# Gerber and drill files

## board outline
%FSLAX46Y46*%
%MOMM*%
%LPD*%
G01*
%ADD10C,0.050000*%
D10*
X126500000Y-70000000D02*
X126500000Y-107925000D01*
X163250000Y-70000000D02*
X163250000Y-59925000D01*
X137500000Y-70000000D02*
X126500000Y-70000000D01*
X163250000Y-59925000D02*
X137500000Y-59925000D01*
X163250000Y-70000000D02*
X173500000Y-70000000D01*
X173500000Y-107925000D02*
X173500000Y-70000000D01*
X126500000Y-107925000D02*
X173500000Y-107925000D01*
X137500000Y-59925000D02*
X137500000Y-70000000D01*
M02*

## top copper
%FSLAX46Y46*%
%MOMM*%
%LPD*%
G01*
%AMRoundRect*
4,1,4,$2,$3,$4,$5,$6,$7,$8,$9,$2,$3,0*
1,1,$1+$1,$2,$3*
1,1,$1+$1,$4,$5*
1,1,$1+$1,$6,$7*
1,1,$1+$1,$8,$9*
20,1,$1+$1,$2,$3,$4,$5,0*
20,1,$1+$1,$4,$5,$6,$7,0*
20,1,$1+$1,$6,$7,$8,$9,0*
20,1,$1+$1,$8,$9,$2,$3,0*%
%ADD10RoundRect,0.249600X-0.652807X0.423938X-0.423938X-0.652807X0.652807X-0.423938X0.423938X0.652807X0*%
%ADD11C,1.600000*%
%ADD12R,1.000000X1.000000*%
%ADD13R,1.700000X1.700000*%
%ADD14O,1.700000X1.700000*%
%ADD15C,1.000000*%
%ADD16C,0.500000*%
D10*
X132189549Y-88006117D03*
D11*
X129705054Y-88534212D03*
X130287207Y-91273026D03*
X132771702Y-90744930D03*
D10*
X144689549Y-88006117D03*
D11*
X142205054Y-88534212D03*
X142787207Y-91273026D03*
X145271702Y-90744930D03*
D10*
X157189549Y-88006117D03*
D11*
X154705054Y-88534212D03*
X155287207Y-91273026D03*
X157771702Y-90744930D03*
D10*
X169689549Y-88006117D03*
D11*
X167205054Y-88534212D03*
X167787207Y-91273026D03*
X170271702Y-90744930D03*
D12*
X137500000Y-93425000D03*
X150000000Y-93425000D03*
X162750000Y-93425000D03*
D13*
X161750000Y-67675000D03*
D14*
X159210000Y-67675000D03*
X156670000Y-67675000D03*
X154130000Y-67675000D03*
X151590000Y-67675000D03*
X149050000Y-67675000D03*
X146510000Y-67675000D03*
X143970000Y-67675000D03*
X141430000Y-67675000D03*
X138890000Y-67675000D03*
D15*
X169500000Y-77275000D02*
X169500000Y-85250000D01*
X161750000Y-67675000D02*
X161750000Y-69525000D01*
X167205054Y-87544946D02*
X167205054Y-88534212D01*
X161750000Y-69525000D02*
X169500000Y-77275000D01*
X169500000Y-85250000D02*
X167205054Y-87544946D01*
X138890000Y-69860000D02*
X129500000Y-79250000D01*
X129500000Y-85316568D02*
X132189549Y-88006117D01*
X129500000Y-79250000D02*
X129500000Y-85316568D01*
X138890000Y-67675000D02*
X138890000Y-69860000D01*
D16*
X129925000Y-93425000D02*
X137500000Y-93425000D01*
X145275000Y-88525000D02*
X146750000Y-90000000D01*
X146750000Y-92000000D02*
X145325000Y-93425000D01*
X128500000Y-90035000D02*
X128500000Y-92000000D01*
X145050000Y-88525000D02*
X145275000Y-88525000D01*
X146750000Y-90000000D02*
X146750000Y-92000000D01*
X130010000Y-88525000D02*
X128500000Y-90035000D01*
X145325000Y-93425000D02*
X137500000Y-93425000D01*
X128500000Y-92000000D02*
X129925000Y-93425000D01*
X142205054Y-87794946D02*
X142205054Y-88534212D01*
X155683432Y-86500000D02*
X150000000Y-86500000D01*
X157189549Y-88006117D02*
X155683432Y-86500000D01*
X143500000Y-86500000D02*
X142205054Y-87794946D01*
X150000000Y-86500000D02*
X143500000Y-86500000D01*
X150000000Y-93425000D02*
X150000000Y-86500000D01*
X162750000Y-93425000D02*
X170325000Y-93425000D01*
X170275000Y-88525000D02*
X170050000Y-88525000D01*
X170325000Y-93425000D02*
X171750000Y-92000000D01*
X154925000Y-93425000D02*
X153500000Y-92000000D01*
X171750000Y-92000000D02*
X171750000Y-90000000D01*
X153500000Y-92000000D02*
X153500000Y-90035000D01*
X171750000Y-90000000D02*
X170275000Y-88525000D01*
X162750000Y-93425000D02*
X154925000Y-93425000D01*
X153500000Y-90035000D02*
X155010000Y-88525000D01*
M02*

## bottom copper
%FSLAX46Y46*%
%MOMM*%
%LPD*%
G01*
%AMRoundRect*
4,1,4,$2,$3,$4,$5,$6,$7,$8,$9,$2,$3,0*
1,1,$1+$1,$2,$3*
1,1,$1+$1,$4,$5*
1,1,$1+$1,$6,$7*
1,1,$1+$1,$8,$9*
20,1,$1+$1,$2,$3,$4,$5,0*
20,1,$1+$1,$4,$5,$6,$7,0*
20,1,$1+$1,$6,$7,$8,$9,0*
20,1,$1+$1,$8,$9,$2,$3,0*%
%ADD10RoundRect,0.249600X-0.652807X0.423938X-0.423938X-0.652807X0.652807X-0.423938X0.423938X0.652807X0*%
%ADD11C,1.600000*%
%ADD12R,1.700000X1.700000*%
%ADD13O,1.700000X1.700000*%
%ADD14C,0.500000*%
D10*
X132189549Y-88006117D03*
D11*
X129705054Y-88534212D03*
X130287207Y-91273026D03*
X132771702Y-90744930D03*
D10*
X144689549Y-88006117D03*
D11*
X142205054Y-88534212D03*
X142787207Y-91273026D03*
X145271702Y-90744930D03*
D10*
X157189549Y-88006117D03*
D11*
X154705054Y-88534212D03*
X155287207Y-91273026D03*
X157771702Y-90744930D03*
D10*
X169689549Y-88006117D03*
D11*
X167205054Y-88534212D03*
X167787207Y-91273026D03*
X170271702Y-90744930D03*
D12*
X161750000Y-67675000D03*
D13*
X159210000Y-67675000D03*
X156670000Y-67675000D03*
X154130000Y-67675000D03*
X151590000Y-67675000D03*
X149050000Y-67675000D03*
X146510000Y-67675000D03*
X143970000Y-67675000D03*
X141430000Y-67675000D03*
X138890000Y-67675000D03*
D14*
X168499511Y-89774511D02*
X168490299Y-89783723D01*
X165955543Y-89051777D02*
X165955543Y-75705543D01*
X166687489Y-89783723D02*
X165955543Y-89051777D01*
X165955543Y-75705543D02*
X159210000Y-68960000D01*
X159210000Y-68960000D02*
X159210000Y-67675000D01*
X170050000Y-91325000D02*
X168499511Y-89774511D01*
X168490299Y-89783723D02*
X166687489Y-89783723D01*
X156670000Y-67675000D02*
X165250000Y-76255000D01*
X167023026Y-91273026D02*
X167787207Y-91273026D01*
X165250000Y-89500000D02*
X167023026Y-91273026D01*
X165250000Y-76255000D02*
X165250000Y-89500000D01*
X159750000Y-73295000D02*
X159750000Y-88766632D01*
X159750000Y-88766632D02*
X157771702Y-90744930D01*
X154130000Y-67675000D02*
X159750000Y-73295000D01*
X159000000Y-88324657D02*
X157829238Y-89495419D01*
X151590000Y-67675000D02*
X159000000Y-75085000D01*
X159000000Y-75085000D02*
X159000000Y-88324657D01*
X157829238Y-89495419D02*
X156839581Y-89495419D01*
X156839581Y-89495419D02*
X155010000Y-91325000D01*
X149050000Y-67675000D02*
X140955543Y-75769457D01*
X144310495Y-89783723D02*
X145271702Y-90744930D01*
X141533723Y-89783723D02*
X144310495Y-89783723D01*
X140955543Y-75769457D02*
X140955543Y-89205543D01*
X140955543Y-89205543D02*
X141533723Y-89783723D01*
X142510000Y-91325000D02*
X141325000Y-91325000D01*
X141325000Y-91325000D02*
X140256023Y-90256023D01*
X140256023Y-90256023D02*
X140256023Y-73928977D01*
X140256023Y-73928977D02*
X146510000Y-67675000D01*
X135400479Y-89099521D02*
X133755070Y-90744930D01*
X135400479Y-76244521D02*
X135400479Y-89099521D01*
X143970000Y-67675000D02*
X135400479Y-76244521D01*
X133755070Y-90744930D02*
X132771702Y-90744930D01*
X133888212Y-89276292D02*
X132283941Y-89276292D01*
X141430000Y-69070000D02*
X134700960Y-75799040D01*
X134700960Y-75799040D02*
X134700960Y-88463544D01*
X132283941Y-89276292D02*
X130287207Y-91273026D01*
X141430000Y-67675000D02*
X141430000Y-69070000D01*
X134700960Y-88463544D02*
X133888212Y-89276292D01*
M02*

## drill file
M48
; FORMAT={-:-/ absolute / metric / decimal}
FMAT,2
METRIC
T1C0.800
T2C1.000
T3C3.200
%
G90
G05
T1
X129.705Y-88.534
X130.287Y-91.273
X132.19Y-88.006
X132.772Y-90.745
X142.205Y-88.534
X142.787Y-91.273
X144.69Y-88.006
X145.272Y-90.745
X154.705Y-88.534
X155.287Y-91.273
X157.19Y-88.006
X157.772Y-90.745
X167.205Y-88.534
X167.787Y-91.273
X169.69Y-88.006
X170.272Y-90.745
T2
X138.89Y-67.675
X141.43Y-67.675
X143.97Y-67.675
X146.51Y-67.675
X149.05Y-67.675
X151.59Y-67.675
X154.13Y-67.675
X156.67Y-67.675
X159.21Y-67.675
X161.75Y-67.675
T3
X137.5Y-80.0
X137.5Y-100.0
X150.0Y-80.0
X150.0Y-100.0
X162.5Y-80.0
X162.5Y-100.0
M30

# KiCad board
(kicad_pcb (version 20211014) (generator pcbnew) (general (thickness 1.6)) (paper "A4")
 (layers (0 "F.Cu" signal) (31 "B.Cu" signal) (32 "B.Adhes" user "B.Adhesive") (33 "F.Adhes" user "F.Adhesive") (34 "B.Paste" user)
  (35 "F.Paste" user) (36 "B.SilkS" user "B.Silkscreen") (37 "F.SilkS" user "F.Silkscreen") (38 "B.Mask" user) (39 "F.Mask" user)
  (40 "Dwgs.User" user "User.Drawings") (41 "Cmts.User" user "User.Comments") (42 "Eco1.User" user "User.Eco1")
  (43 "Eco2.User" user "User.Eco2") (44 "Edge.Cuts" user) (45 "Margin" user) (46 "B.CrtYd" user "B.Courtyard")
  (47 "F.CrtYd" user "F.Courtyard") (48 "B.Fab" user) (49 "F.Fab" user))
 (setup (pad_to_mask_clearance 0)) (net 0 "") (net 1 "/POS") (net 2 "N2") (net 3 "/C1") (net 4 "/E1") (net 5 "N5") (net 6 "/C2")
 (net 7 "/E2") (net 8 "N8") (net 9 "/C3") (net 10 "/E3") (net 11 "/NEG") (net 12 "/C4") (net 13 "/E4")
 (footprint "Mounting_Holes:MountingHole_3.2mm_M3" (layer "F.Cu") (at 137.5 100)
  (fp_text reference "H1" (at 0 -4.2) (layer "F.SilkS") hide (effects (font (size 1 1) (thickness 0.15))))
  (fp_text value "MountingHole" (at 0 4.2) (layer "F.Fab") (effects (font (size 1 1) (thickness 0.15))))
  (pad "" np_thru_hole circle locked (at 0 0) (size 3.2 3.2) (drill 3.2) (layers *.Cu *.Mask)))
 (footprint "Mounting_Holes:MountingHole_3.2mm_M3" (layer "F.Cu") (at 137.5 80)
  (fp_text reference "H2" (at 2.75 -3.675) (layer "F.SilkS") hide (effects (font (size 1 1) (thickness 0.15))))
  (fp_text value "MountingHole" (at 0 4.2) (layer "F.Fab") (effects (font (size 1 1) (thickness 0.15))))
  (pad "" np_thru_hole circle locked (at 0 0) (size 3.2 3.2) (drill 3.2) (layers *.Cu *.Mask)))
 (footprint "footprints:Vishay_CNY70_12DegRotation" (layer "F.Cu") (at 131.15 89.795 -90)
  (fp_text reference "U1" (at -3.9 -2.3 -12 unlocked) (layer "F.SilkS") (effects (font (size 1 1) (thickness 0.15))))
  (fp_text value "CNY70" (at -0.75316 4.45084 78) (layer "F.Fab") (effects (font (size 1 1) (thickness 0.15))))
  (pad "1" thru_hole roundrect (at -1.788883 -1.039549 282) (size 1.6 1.6) (drill 0.8) (layers *.Cu *.Mask) (roundrect_rratio 0.156)
   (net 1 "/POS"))
  (pad "2" thru_hole circle (at -1.260788 1.444946 282) (size 1.6 1.6) (drill 0.8) (layers *.Cu *.Mask) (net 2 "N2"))
  (pad "3" thru_hole circle (at 1.478026 0.862793 282) (size 1.6 1.6) (drill 0.8) (layers *.Cu *.Mask) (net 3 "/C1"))
  (pad "4" thru_hole circle (at 0.94993 -1.621702 282) (size 1.6 1.6) (drill 0.8) (layers *.Cu *.Mask) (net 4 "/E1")))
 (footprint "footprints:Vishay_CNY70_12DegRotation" (layer "F.Cu") (at 143.65 89.795 -90)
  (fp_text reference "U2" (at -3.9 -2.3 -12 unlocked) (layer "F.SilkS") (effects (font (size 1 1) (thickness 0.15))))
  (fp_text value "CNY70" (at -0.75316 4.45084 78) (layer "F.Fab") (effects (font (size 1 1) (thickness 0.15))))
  (pad "1" thru_hole roundrect (at -1.788883 -1.039549 282) (size 1.6 1.6) (drill 0.8) (layers *.Cu *.Mask) (roundrect_rratio 0.156)
   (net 2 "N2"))
  (pad "2" thru_hole circle (at -1.260788 1.444946 282) (size 1.6 1.6) (drill 0.8) (layers *.Cu *.Mask) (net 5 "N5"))
  (pad "3" thru_hole circle (at 1.478026 0.862793 282) (size 1.6 1.6) (drill 0.8) (layers *.Cu *.Mask) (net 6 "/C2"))
  (pad "4" thru_hole circle (at 0.94993 -1.621702 282) (size 1.6 1.6) (drill 0.8) (layers *.Cu *.Mask) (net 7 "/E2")))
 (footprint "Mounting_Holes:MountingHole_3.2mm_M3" (layer "F.Cu") (at 150 100)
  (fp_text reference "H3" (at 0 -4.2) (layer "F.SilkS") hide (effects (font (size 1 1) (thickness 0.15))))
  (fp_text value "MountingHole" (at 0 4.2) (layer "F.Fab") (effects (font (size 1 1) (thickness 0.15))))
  (pad "" np_thru_hole circle locked (at 0 0) (size 3.2 3.2) (drill 3.2) (layers *.Cu *.Mask)))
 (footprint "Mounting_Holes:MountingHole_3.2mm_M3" (layer "F.Cu") (at 150 80)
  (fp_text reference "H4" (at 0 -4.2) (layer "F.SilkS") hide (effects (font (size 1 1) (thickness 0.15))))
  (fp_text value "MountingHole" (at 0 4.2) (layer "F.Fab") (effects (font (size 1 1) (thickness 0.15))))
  (pad "" np_thru_hole circle locked (at 0 0) (size 3.2 3.2) (drill 3.2) (layers *.Cu *.Mask)))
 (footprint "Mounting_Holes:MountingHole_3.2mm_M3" (layer "F.Cu") (at 162.5 100)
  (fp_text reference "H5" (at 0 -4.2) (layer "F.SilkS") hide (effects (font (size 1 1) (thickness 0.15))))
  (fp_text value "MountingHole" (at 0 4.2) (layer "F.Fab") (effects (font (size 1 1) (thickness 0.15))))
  (pad "" np_thru_hole circle locked (at 0 0) (size 3.2 3.2) (drill 3.2) (layers *.Cu *.Mask)))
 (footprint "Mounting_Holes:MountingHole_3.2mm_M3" (layer "F.Cu") (at 162.5 80)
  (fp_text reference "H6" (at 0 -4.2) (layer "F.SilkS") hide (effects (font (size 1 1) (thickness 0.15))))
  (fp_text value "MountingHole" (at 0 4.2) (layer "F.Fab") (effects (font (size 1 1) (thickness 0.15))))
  (pad "" np_thru_hole circle locked (at 0 0) (size 3.2 3.2) (drill 3.2) (layers *.Cu *.Mask)))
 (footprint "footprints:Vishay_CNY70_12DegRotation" (layer "F.Cu") (at 156.15 89.795 -90)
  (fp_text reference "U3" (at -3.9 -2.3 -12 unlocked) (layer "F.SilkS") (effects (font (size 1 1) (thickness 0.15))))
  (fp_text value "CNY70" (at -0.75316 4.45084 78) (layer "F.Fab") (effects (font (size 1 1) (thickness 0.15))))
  (pad "1" thru_hole roundrect (at -1.788883 -1.039549 282) (size 1.6 1.6) (drill 0.8) (layers *.Cu *.Mask) (roundrect_rratio 0.156)
   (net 5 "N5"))
  (pad "2" thru_hole circle (at -1.260788 1.444946 282) (size 1.6 1.6) (drill 0.8) (layers *.Cu *.Mask) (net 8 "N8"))
  (pad "3" thru_hole circle (at 1.478026 0.862793 282) (size 1.6 1.6) (drill 0.8) (layers *.Cu *.Mask) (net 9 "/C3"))
  (pad "4" thru_hole circle (at 0.94993 -1.621702 282) (size 1.6 1.6) (drill 0.8) (layers *.Cu *.Mask) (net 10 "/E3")))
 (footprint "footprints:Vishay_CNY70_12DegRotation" (layer "F.Cu") (at 168.65 89.795 -90)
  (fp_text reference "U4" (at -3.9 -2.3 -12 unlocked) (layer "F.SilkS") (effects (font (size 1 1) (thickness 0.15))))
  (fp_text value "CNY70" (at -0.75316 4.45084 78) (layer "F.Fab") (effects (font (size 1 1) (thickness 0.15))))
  (pad "1" thru_hole roundrect (at -1.788883 -1.039549 282) (size 1.6 1.6) (drill 0.8) (layers *.Cu *.Mask) (roundrect_rratio 0.156)
   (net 8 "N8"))
  (pad "2" thru_hole circle (at -1.260788 1.444946 282) (size 1.6 1.6) (drill 0.8) (layers *.Cu *.Mask) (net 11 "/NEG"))
  (pad "3" thru_hole circle (at 1.478026 0.862793 282) (size 1.6 1.6) (drill 0.8) (layers *.Cu *.Mask) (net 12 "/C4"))
  (pad "4" thru_hole circle (at 0.94993 -1.621702 282) (size 1.6 1.6) (drill 0.8) (layers *.Cu *.Mask) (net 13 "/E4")))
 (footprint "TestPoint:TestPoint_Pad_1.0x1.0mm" (layer "F.Cu") (at 137.5 93.425)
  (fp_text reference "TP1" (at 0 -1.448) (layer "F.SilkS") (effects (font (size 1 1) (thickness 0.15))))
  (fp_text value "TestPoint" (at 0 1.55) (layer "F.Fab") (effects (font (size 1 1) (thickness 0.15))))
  (pad "1" smd rect locked (at 0 0) (size 1 1) (layers "F.Cu" "F.Mask") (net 2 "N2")))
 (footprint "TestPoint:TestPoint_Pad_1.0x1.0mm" (layer "F.Cu") (at 150 93.425)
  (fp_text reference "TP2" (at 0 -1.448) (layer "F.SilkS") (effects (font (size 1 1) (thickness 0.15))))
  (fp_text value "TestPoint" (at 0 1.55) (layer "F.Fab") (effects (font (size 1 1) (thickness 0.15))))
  (pad "1" smd rect locked (at 0 0) (size 1 1) (layers "F.Cu" "F.Mask") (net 5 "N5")))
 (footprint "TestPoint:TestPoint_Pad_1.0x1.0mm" (layer "F.Cu") (at 162.75 93.425)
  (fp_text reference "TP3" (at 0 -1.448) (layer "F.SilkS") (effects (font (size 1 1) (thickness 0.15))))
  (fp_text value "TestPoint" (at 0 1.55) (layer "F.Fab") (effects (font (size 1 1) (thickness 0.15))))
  (pad "1" smd rect locked (at 0 0) (size 1 1) (layers "F.Cu" "F.Mask") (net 8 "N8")))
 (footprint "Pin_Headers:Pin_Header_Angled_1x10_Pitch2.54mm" (layer "B.Cu") (at 161.75 67.675 90)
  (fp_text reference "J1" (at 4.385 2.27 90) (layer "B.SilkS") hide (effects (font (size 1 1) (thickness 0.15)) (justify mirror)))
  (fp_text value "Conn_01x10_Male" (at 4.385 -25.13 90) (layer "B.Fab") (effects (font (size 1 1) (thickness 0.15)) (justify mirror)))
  (pad "1" thru_hole rect (at 0 0 90) (size 1.7 1.7) (drill 1) (layers *.Cu *.Mask) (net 11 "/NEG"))
  (pad "2" thru_hole oval (at 0 -2.54 90) (size 1.7 1.7) (drill 1) (layers *.Cu *.Mask) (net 13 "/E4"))
  (pad "3" thru_hole oval (at 0 -5.08 90) (size 1.7 1.7) (drill 1) (layers *.Cu *.Mask) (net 12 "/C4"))
  (pad "4" thru_hole oval (at 0 -7.62 90) (size 1.7 1.7) (drill 1) (layers *.Cu *.Mask) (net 10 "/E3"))
  (pad "5" thru_hole oval (at 0 -10.16 90) (size 1.7 1.7) (drill 1) (layers *.Cu *.Mask) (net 9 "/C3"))
  (pad "6" thru_hole oval (at 0 -12.7 90) (size 1.7 1.7) (drill 1) (layers *.Cu *.Mask) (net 7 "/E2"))
  (pad "7" thru_hole oval (at 0 -15.24 90) (size 1.7 1.7) (drill 1) (layers *.Cu *.Mask) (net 6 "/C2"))
  (pad "8" thru_hole oval (at 0 -17.78 90) (size 1.7 1.7) (drill 1) (layers *.Cu *.Mask) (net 4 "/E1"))
  (pad "9" thru_hole oval (at 0 -20.32 90) (size 1.7 1.7) (drill 1) (layers *.Cu *.Mask) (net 3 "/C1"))
  (pad "10" thru_hole oval (at 0 -22.86 90) (size 1.7 1.7) (drill 1) (layers *.Cu *.Mask) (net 1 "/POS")))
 (gr_line (start 126.5 70) (end 126.5 107.925) (layer "Edge.Cuts") (width 0.05))
 (gr_line (start 163.25 70) (end 163.25 59.925) (layer "Edge.Cuts") (width 0.05))
 (gr_line (start 137.5 70) (end 126.5 70) (layer "Edge.Cuts") (width 0.05))
 (gr_line (start 163.25 59.925) (end 137.5 59.925) (layer "Edge.Cuts") (width 0.05))
 (gr_line (start 163.25 70) (end 173.5 70) (layer "Edge.Cuts") (width 0.05))
 (gr_line (start 173.5 107.925) (end 173.5 70) (layer "Edge.Cuts") (width 0.05))
 (gr_line (start 126.5 107.925) (end 173.5 107.925) (layer "Edge.Cuts") (width 0.05))
 (gr_line (start 137.5 59.925) (end 137.5 70) (layer "Edge.Cuts") (width 0.05))
 (segment (start 169.5 77.275) (end 169.5 85.25) (width 1) (layer "F.Cu") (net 11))
 (segment (start 161.75 67.675) (end 161.75 69.525) (width 1) (layer "F.Cu") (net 11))
 (segment (start 167.205054 87.544946) (end 167.205054 88.534212) (width 1) (layer "F.Cu") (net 11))
 (segment (start 161.75 69.525) (end 169.5 77.275) (width 1) (layer "F.Cu") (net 11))
 (segment (start 169.5 85.25) (end 167.205054 87.544946) (width 1) (layer "F.Cu") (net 11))
 (segment (start 138.89 69.86) (end 129.5 79.25) (width 1) (layer "F.Cu") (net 1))
 (segment (start 129.5 85.316568) (end 132.189549 88.006117) (width 1) (layer "F.Cu") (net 1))
 (segment (start 129.5 79.25) (end 129.5 85.316568) (width 1) (layer "F.Cu") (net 1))
 (segment (start 138.89 67.675) (end 138.89 69.86) (width 1) (layer "F.Cu") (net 1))
 (segment (start 168.499511 89.774511) (end 168.490299 89.783723) (width 0.5) (layer "B.Cu") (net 13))
 (segment (start 165.955543 89.051777) (end 165.955543 75.705543) (width 0.5) (layer "B.Cu") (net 13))
 (segment (start 166.687489 89.783723) (end 165.955543 89.051777) (width 0.5) (layer "B.Cu") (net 13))
 (segment (start 165.955543 75.705543) (end 159.21 68.96) (width 0.5) (layer "B.Cu") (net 13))
 (segment (start 159.21 68.96) (end 159.21 67.675) (width 0.5) (layer "B.Cu") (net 13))
 (segment (start 170.05 91.325) (end 168.499511 89.774511) (width 0.5) (layer "B.Cu") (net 13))
 (segment (start 168.490299 89.783723) (end 166.687489 89.783723) (width 0.5) (layer "B.Cu") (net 13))
 (segment (start 156.67 67.675) (end 165.25 76.255) (width 0.5) (layer "B.Cu") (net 12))
 (segment (start 167.023026 91.273026) (end 167.787207 91.273026) (width 0.5) (layer "B.Cu") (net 12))
 (segment (start 165.25 89.5) (end 167.023026 91.273026) (width 0.5) (layer "B.Cu") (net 12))
 (segment (start 165.25 76.255) (end 165.25 89.5) (width 0.5) (layer "B.Cu") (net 12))
 (segment (start 159.75 73.295) (end 159.75 88.766632) (width 0.5) (layer "B.Cu") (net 10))
 (segment (start 159.75 88.766632) (end 157.771702 90.74493) (width 0.5) (layer "B.Cu") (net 10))
 (segment (start 154.13 67.675) (end 159.75 73.295) (width 0.5) (layer "B.Cu") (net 10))
 (segment (start 159 88.324657) (end 157.829238 89.495419) (width 0.5) (layer "B.Cu") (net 9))
 (segment (start 151.59 67.675) (end 159 75.085) (width 0.5) (layer "B.Cu") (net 9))
 (segment (start 159 75.085) (end 159 88.324657) (width 0.5) (layer "B.Cu") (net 9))
 (segment (start 157.829238 89.495419) (end 156.839581 89.495419) (width 0.5) (layer "B.Cu") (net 9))
 (segment (start 156.839581 89.495419) (end 155.01 91.325) (width 0.5) (layer "B.Cu") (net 9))
 (segment (start 149.05 67.675) (end 140.955543 75.769457) (width 0.5) (layer "B.Cu") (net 7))
 (segment (start 144.310495 89.783723) (end 145.271702 90.74493) (width 0.5) (layer "B.Cu") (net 7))
 (segment (start 141.533723 89.783723) (end 144.310495 89.783723) (width 0.5) (layer "B.Cu") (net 7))
 (segment (start 140.955543 75.769457) (end 140.955543 89.205543) (width 0.5) (layer "B.Cu") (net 7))
 (segment (start 140.955543 89.205543) (end 141.533723 89.783723) (width 0.5) (layer "B.Cu") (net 7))
 (segment (start 142.51 91.325) (end 141.325 91.325) (width 0.5) (layer "B.Cu") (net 6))
 (segment (start 141.325 91.325) (end 140.256023 90.256023) (width 0.5) (layer "B.Cu") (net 6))
 (segment (start 140.256023 90.256023) (end 140.256023 73.928977) (width 0.5) (layer "B.Cu") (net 6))
 (segment (start 140.256023 73.928977) (end 146.51 67.675) (width 0.5) (layer "B.Cu") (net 6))
 (segment (start 135.400479 89.099521) (end 133.75507 90.74493) (width 0.5) (layer "B.Cu") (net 4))
 (segment (start 135.400479 76.244521) (end 135.400479 89.099521) (width 0.5) (layer "B.Cu") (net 4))
 (segment (start 143.97 67.675) (end 135.400479 76.244521) (width 0.5) (layer "B.Cu") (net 4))
 (segment (start 133.75507 90.74493) (end 132.771702 90.74493) (width 0.5) (layer "B.Cu") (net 4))
 (segment (start 133.888212 89.276292) (end 132.283941 89.276292) (width 0.5) (layer "B.Cu") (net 3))
 (segment (start 141.43 69.07) (end 134.70096 75.79904) (width 0.5) (layer "B.Cu") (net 3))
 (segment (start 134.70096 75.79904) (end 134.70096 88.463544) (width 0.5) (layer "B.Cu") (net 3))
 (segment (start 132.283941 89.276292) (end 130.287207 91.273026) (width 0.5) (layer "B.Cu") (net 3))
 (segment (start 141.43 67.675) (end 141.43 69.07) (width 0.5) (layer "B.Cu") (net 3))
 (segment (start 134.70096 88.463544) (end 133.888212 89.276292) (width 0.5) (layer "B.Cu") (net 3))
 (segment (start 129.925 93.425) (end 137.5 93.425) (width 0.5) (layer "F.Cu") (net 2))
 (segment (start 145.275 88.525) (end 146.75 90) (width 0.5) (layer "F.Cu") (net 2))
 (segment (start 146.75 92) (end 145.325 93.425) (width 0.5) (layer "F.Cu") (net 2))
 (segment (start 128.5 90.035) (end 128.5 92) (width 0.5) (layer "F.Cu") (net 2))
 (segment (start 145.05 88.525) (end 145.275 88.525) (width 0.5) (layer "F.Cu") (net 2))
 (segment (start 146.75 90) (end 146.75 92) (width 0.5) (layer "F.Cu") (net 2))
 (segment (start 130.01 88.525) (end 128.5 90.035) (width 0.5) (layer "F.Cu") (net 2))
 (segment (start 145.325 93.425) (end 137.5 93.425) (width 0.5) (layer "F.Cu") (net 2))
 (segment (start 128.5 92) (end 129.925 93.425) (width 0.5) (layer "F.Cu") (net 2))
 (segment (start 142.205054 87.794946) (end 142.205054 88.534212) (width 0.5) (layer "F.Cu") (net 5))
 (segment (start 155.683432 86.5) (end 150 86.5) (width 0.5) (layer "F.Cu") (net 5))
 (segment (start 157.189549 88.006117) (end 155.683432 86.5) (width 0.5) (layer "F.Cu") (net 5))
 (segment (start 143.5 86.5) (end 142.205054 87.794946) (width 0.5) (layer "F.Cu") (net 5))
 (segment (start 150 86.5) (end 143.5 86.5) (width 0.5) (layer "F.Cu") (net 5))
 (segment (start 150 93.425) (end 150 86.5) (width 0.5) (layer "F.Cu") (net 5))
 (segment (start 162.75 93.425) (end 170.325 93.425) (width 0.5) (layer "F.Cu") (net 8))
 (segment (start 170.275 88.525) (end 170.05 88.525) (width 0.5) (layer "F.Cu") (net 8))
 (segment (start 170.325 93.425) (end 171.75 92) (width 0.5) (layer "F.Cu") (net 8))
 (segment (start 154.925 93.425) (end 153.5 92) (width 0.5) (layer "F.Cu") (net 8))
 (segment (start 171.75 92) (end 171.75 90) (width 0.5) (layer "F.Cu") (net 8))
 (segment (start 153.5 92) (end 153.5 90.035) (width 0.5) (layer "F.Cu") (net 8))
 (segment (start 171.75 90) (end 170.275 88.525) (width 0.5) (layer "F.Cu") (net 8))
 (segment (start 162.75 93.425) (end 154.925 93.425) (width 0.5) (layer "F.Cu") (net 8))
 (segment (start 153.5 90.035) (end 155.01 88.525) (width 0.5) (layer "F.Cu") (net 8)))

